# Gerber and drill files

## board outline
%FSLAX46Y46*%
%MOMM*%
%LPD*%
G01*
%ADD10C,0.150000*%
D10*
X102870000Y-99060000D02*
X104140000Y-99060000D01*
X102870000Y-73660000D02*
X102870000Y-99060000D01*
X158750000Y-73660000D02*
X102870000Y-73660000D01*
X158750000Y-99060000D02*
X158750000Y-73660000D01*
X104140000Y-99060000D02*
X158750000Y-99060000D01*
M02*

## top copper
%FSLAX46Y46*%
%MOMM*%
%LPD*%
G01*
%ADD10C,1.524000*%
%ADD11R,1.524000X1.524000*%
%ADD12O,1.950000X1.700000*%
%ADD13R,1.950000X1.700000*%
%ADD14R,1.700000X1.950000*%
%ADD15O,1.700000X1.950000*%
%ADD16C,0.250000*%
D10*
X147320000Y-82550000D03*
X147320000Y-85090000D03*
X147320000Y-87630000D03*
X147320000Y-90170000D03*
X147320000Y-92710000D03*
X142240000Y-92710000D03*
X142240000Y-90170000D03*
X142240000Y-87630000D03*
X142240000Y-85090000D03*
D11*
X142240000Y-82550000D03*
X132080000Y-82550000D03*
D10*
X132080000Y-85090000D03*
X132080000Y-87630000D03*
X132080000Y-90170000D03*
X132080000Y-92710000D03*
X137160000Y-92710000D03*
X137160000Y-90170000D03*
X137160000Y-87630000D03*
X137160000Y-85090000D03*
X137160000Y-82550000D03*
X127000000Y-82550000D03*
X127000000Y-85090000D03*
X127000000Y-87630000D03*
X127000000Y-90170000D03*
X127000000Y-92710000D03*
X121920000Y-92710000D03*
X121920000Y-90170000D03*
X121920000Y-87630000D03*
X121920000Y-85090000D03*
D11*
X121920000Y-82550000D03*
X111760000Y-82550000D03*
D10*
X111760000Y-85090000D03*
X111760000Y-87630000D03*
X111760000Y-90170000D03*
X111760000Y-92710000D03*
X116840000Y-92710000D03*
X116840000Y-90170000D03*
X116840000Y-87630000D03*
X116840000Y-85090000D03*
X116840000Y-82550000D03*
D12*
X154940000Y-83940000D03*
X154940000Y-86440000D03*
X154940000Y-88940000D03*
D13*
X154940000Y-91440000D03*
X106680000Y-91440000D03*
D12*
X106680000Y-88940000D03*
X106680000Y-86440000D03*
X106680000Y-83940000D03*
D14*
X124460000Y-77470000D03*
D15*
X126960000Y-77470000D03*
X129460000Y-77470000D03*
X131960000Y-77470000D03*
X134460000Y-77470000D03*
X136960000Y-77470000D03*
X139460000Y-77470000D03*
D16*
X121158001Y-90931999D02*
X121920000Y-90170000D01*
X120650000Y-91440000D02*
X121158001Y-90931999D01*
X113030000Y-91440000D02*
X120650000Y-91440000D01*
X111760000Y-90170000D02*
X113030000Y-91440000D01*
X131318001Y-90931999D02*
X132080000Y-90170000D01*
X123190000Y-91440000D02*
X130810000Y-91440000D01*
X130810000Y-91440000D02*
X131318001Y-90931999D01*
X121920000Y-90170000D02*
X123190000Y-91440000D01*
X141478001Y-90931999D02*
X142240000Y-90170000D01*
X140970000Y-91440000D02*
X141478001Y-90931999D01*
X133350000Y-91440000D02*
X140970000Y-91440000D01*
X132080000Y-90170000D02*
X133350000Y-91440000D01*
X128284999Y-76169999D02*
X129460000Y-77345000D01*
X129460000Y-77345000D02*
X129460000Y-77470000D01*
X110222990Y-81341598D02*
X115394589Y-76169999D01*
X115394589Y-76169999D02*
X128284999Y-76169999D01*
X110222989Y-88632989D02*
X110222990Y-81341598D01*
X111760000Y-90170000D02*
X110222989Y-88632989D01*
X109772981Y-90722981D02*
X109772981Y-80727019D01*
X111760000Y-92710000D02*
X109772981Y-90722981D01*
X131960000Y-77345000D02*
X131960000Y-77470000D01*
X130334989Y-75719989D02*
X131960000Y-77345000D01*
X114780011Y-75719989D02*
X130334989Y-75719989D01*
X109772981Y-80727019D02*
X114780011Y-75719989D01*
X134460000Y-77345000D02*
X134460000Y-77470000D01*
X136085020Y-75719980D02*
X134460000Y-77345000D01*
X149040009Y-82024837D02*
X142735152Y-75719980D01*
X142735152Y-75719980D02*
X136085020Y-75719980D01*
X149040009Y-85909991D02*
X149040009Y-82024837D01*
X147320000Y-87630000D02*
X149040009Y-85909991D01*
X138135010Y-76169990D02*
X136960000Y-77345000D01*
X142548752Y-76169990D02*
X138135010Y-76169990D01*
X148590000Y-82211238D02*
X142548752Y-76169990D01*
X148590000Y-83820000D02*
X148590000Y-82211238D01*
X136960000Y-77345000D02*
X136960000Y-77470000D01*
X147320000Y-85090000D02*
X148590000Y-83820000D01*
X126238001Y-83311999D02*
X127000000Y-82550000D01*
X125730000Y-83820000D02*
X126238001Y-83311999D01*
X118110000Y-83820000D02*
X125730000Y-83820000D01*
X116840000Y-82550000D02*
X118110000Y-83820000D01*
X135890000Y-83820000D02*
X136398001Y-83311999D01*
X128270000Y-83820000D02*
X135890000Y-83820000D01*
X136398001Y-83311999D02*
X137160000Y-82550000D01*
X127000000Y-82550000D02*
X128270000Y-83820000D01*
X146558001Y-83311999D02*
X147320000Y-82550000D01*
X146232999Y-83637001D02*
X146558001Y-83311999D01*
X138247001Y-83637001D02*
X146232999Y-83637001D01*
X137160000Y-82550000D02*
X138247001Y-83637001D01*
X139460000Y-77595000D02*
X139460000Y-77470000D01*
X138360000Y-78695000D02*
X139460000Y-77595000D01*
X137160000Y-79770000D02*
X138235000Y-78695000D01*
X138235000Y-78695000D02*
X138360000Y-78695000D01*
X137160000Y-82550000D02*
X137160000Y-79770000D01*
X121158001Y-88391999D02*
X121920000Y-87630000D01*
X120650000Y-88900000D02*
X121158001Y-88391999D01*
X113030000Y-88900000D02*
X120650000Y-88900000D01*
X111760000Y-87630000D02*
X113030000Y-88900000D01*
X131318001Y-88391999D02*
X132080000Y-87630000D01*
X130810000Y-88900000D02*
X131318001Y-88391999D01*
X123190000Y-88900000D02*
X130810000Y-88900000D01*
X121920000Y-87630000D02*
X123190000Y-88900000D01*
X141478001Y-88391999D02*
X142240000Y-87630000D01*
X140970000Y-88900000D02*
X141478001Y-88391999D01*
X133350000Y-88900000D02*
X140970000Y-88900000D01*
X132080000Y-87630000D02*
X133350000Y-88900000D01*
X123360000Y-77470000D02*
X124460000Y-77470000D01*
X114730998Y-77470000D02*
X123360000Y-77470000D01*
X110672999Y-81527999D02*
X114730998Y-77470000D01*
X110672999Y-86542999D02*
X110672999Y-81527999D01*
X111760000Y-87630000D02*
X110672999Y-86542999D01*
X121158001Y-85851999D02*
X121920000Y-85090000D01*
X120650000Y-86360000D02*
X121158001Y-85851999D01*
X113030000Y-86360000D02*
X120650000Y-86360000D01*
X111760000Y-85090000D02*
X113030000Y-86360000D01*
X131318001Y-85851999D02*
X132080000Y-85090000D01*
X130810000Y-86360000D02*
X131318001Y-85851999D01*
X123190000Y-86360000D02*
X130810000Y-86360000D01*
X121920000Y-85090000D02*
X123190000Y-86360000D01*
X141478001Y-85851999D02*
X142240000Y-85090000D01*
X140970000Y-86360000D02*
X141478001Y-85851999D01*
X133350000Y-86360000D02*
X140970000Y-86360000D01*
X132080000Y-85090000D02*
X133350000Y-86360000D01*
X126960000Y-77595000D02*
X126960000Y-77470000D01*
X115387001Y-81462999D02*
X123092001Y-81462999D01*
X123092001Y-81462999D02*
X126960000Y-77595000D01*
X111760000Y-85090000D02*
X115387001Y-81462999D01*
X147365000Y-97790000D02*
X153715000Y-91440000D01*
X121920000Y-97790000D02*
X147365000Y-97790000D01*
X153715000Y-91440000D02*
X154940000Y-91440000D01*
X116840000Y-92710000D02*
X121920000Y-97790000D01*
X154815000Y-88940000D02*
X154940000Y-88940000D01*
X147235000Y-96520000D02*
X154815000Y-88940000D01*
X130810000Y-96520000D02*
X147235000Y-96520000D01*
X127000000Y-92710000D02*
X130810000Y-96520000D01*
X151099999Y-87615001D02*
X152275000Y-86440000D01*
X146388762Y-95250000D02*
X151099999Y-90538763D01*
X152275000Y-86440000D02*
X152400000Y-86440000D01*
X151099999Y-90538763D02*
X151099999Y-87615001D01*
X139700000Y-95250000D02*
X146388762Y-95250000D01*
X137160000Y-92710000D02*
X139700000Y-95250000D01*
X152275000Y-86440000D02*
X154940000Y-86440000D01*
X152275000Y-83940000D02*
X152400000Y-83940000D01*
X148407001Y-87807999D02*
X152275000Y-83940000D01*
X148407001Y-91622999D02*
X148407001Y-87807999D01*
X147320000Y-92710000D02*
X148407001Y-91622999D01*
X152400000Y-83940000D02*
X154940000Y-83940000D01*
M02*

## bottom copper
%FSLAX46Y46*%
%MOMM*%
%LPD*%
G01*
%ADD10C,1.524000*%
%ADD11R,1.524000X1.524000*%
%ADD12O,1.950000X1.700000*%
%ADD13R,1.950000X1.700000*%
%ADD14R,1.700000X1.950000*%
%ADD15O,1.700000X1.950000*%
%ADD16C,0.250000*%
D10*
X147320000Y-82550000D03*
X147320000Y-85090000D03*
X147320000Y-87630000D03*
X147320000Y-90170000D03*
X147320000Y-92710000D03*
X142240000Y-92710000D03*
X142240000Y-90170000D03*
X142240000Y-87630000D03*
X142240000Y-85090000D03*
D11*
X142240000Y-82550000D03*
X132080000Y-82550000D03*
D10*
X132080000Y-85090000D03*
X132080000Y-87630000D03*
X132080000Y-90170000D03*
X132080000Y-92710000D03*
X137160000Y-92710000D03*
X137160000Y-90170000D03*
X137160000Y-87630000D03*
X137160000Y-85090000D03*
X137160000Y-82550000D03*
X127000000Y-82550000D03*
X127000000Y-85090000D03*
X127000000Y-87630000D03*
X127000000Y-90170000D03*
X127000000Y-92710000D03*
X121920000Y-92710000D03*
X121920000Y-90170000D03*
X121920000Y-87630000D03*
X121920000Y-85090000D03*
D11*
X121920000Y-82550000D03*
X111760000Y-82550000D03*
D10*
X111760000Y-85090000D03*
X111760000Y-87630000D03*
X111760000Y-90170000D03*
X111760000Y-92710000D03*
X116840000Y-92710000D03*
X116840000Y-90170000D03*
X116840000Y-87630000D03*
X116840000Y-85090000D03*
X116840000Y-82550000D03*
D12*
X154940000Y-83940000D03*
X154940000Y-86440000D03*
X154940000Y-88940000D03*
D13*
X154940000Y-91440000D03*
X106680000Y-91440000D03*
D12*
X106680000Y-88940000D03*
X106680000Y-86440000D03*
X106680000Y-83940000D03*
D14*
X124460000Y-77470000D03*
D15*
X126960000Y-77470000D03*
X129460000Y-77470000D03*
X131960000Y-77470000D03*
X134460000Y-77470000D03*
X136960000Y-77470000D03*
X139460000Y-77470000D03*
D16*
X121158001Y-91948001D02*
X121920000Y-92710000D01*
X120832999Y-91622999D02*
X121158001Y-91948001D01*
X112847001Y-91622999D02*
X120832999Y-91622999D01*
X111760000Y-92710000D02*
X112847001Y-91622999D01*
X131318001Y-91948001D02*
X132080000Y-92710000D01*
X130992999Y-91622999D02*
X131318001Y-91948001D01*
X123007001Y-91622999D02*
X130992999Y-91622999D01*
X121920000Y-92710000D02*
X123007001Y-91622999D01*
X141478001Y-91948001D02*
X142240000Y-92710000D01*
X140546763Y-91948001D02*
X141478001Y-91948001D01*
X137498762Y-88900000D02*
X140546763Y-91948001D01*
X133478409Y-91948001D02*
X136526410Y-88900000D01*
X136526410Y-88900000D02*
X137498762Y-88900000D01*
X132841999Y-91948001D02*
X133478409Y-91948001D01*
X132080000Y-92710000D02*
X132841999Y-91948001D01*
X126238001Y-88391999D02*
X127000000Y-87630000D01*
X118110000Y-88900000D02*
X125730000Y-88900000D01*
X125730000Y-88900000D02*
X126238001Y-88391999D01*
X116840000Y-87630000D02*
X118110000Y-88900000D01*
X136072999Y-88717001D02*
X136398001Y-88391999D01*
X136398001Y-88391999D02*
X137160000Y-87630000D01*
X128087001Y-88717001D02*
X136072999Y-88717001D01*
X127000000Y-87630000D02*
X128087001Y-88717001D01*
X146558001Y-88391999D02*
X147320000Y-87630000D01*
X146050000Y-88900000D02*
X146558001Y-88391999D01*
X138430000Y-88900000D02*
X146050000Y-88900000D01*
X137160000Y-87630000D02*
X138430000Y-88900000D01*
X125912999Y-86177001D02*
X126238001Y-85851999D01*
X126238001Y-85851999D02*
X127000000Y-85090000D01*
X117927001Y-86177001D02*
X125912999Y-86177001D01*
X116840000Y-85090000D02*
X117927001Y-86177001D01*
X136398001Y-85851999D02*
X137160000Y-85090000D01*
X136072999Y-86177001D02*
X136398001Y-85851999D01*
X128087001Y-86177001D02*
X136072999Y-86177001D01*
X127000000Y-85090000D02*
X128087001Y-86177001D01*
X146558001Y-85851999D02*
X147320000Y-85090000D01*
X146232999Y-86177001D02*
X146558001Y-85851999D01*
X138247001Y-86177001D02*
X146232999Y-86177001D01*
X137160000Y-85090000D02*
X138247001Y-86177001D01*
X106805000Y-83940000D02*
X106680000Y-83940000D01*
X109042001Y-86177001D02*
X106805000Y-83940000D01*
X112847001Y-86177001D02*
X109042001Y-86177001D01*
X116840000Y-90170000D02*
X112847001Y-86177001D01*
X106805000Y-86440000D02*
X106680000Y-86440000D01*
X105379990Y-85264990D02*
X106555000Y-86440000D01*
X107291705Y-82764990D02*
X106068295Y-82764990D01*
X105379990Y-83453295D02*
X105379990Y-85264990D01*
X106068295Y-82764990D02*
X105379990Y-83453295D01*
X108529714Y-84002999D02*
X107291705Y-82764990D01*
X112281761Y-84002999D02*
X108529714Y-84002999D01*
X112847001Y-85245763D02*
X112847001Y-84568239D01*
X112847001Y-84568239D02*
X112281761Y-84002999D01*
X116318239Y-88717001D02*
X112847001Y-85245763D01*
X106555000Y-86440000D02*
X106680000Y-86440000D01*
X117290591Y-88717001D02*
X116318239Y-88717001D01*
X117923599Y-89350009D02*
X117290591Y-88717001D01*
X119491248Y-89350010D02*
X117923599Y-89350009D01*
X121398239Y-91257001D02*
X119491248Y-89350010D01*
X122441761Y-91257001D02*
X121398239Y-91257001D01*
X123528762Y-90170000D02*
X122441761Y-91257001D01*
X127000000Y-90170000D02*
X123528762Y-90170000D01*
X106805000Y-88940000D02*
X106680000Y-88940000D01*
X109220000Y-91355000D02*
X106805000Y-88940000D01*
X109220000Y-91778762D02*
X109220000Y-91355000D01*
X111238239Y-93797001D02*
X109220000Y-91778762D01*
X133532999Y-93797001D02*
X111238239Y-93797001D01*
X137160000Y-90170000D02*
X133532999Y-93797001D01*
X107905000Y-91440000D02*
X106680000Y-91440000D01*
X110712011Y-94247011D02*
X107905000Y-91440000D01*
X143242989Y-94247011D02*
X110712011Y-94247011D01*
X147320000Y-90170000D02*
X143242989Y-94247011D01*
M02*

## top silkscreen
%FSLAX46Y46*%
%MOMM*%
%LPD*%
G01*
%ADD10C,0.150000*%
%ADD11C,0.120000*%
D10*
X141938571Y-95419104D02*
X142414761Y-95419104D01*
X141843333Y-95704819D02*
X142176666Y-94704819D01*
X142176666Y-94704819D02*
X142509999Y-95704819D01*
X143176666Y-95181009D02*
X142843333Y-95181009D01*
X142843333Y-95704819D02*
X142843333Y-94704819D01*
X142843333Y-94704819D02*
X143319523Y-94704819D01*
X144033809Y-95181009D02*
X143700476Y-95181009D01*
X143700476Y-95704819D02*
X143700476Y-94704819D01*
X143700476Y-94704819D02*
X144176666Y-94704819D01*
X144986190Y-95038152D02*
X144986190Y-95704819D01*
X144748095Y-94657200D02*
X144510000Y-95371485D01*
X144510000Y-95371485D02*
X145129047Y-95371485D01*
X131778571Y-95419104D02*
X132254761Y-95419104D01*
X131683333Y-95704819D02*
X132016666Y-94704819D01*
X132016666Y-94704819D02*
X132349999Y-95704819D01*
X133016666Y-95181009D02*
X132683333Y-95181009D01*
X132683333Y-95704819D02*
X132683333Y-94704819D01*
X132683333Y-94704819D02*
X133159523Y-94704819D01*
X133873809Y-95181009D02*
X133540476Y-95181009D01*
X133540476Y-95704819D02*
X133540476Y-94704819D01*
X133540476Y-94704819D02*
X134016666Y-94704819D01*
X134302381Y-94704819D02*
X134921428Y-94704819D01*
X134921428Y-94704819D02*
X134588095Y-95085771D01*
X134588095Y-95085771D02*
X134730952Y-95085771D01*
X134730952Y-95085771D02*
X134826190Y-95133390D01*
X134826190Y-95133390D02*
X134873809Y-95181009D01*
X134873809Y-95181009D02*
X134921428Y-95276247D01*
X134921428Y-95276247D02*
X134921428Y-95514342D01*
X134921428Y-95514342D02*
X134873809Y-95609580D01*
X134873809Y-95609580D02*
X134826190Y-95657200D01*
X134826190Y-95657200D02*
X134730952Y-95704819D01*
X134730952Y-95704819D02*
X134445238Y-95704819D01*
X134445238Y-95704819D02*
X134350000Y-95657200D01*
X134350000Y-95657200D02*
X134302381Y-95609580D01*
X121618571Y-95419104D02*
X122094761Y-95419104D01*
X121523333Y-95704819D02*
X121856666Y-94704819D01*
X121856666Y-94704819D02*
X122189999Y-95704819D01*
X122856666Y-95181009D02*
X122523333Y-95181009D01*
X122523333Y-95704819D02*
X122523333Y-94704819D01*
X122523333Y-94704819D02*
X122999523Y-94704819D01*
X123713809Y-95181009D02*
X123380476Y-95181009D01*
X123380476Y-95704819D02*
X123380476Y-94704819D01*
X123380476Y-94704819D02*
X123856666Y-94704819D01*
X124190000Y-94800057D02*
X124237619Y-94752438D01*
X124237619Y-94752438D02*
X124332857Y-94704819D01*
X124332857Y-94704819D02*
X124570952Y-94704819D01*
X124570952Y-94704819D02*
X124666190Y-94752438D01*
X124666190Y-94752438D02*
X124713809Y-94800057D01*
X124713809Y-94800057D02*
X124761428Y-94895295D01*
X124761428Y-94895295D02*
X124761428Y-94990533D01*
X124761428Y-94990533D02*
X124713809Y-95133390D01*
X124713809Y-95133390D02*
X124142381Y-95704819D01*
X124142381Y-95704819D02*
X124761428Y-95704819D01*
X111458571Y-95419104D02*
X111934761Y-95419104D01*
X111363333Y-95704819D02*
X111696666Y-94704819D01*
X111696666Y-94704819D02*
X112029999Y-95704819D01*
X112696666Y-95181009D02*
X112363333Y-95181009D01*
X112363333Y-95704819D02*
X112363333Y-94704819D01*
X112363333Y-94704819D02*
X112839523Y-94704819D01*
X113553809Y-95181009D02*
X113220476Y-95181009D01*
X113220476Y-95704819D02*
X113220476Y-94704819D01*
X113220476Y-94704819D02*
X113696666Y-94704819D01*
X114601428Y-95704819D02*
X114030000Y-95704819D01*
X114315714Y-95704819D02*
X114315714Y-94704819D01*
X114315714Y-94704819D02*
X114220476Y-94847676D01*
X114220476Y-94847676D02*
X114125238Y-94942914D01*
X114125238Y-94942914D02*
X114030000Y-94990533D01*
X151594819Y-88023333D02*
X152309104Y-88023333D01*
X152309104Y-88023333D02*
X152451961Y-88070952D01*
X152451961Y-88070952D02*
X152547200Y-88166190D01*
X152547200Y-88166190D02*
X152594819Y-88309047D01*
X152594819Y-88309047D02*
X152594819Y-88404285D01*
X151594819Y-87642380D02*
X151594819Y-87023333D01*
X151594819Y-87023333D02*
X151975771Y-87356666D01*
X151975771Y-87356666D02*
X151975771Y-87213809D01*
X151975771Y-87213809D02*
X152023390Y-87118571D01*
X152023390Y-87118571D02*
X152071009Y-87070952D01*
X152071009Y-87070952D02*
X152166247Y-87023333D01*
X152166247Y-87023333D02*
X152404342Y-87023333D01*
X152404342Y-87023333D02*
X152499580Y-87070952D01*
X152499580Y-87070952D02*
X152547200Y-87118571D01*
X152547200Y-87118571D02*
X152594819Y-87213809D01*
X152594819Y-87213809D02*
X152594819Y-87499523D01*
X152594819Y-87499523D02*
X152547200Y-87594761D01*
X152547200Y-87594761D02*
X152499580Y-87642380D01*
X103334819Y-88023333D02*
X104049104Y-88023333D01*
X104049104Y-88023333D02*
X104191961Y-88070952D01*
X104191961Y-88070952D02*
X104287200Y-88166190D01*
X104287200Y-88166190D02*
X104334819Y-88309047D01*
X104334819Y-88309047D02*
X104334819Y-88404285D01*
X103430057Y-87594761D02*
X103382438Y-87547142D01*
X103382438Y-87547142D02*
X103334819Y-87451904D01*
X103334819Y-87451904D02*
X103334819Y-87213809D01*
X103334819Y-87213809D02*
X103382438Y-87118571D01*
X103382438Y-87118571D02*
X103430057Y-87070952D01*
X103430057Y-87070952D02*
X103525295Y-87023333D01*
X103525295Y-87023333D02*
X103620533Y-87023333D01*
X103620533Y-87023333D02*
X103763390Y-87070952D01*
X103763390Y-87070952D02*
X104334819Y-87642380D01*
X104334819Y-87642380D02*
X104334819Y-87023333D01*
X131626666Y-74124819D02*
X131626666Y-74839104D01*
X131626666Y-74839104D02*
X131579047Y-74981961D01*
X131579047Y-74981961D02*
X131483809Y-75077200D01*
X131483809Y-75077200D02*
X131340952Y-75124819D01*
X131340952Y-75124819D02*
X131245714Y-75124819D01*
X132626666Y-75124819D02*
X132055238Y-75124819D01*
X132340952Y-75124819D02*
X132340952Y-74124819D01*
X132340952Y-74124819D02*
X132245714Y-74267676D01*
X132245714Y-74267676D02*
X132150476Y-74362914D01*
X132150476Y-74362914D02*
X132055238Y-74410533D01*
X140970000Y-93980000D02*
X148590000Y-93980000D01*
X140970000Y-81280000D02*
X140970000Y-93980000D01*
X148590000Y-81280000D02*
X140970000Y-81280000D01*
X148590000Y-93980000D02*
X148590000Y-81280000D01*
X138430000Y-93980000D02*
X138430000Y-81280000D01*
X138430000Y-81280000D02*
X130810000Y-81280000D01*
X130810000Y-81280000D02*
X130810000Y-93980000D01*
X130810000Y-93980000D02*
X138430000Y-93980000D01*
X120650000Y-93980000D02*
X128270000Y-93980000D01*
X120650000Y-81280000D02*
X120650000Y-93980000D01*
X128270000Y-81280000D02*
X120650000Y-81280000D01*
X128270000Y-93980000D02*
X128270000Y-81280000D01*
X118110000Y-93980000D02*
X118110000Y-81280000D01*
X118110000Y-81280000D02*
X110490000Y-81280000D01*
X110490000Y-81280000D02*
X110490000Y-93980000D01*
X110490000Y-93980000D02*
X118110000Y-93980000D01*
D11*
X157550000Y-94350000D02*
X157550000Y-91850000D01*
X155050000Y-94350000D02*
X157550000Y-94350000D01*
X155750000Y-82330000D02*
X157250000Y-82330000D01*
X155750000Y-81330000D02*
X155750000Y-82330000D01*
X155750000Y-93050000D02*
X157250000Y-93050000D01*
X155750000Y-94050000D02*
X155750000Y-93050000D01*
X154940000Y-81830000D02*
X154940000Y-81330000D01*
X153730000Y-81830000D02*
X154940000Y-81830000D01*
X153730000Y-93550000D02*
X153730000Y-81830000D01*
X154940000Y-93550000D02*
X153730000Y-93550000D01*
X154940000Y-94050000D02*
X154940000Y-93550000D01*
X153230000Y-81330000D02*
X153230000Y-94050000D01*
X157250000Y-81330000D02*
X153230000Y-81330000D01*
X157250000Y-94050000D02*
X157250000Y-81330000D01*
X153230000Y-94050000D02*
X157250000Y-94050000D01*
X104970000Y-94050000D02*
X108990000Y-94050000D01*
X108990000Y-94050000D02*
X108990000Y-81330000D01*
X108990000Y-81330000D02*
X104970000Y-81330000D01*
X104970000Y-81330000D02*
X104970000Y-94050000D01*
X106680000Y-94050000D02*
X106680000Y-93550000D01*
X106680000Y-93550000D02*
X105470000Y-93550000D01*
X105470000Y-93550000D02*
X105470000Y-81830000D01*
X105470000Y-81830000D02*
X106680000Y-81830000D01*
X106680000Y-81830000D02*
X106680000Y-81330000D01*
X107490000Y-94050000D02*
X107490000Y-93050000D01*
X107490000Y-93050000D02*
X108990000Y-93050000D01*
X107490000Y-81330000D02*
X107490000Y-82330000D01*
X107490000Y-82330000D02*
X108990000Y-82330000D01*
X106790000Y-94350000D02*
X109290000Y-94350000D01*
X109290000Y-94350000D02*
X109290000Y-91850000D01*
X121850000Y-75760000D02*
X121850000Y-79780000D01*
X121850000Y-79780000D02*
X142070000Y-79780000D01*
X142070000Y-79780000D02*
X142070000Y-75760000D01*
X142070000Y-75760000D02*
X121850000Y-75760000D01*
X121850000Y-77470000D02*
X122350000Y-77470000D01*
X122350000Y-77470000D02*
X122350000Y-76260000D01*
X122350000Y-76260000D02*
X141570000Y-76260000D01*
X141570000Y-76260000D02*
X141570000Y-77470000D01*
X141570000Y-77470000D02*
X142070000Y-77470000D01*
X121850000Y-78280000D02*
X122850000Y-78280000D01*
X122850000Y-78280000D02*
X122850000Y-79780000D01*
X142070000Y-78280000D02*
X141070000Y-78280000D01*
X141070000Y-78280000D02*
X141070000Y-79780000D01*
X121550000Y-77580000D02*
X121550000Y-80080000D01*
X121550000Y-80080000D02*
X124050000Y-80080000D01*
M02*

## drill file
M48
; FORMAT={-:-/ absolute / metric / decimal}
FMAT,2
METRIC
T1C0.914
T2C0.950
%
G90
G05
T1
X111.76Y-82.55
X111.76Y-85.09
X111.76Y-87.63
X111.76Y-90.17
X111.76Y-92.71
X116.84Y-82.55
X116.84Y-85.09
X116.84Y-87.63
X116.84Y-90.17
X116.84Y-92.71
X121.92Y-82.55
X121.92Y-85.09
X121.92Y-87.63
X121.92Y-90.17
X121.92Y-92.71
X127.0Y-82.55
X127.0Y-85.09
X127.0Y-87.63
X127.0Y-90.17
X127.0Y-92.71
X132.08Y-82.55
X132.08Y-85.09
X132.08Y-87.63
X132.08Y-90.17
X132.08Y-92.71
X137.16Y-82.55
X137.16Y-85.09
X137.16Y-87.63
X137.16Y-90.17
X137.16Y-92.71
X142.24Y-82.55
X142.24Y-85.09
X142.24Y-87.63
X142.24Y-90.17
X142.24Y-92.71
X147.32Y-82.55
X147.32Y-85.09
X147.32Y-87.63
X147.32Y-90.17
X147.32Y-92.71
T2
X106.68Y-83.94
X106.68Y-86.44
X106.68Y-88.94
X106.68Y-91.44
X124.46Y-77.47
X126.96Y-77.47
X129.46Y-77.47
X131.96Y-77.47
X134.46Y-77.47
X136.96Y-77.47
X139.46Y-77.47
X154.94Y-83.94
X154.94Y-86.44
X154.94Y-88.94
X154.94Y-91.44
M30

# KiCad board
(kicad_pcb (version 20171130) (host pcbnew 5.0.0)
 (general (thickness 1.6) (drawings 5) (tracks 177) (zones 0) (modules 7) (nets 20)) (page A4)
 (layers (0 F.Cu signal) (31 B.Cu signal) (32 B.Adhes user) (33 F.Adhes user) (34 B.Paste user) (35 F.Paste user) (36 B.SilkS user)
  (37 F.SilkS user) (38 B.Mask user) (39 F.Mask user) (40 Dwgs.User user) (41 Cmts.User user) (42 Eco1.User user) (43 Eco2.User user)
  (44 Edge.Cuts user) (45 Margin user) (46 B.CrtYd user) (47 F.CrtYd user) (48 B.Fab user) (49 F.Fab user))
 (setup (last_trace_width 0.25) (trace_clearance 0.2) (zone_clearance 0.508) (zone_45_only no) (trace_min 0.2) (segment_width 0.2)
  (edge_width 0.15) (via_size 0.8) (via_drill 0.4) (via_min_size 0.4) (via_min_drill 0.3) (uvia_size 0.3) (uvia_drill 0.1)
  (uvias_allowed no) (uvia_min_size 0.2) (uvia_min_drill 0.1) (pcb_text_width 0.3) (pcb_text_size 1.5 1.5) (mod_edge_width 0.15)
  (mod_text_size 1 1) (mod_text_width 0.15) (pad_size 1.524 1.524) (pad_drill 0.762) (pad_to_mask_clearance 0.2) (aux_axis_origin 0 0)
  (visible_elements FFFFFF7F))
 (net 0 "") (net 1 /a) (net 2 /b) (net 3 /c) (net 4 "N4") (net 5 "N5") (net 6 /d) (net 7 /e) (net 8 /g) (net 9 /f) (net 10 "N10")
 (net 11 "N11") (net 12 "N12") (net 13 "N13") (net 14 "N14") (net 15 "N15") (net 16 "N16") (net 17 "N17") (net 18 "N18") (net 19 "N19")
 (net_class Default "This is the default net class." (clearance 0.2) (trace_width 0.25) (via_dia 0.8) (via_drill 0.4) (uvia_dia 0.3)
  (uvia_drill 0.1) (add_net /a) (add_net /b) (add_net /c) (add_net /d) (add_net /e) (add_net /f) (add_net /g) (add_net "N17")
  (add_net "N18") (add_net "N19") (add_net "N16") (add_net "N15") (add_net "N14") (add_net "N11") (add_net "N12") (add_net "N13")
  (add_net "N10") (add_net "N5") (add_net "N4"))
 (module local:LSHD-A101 (layer F.Cu) (at 144.78 87.63 90)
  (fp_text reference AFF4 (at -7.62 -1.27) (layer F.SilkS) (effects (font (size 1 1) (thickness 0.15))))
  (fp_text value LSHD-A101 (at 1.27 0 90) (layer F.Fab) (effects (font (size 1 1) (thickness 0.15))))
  (fp_line (start -6.35 -3.81) (end -6.35 3.81) (layer F.SilkS) (width 0.15))
  (fp_line (start 6.35 -3.81) (end -6.35 -3.81) (layer F.SilkS) (width 0.15))
  (fp_line (start 6.35 3.81) (end 6.35 -3.81) (layer F.SilkS) (width 0.15))
  (fp_line (start -6.35 3.81) (end 6.35 3.81) (layer F.SilkS) (width 0.15))
  (pad 10 thru_hole circle (at 5.08 2.54) (size 1.524 1.524) (drill 0.9144) (layers *.Cu *.Mask) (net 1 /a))
  (pad 9 thru_hole circle (at 2.54 2.54) (size 1.524 1.524) (drill 0.9144) (layers *.Cu *.Mask) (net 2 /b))
  (pad 8 thru_hole circle (at 0 2.54) (size 1.524 1.524) (drill 0.9144) (layers *.Cu *.Mask) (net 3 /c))
  (pad 7 thru_hole circle (at -2.54 2.54) (size 1.524 1.524) (drill 0.9144) (layers *.Cu *.Mask) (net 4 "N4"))
  (pad 6 thru_hole circle (at -5.08 2.54) (size 1.524 1.524) (drill 0.9144) (layers *.Cu *.Mask) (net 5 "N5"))
  (pad 5 thru_hole circle (at -5.08 -2.54) (size 1.524 1.524) (drill 0.9144) (layers *.Cu *.Mask) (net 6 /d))
  (pad 4 thru_hole circle (at -2.54 -2.54) (size 1.524 1.524) (drill 0.9144) (layers *.Cu *.Mask) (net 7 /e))
  (pad 3 thru_hole circle (at 0 -2.54) (size 1.524 1.524) (drill 0.9144) (layers *.Cu *.Mask) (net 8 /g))
  (pad 2 thru_hole circle (at 2.54 -2.54) (size 1.524 1.524) (drill 0.9144) (layers *.Cu *.Mask) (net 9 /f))
  (pad 1 thru_hole rect (at 5.08 -2.54) (size 1.524 1.524) (drill 0.9144) (layers *.Cu *.Mask) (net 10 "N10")))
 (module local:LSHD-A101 (layer F.Cu) (at 134.62 87.63 90)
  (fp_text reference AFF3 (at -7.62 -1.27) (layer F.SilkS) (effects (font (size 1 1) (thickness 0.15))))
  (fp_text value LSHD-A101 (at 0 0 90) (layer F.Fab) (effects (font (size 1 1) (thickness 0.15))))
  (fp_line (start -6.35 3.81) (end 6.35 3.81) (layer F.SilkS) (width 0.15))
  (fp_line (start 6.35 3.81) (end 6.35 -3.81) (layer F.SilkS) (width 0.15))
  (fp_line (start 6.35 -3.81) (end -6.35 -3.81) (layer F.SilkS) (width 0.15))
  (fp_line (start -6.35 -3.81) (end -6.35 3.81) (layer F.SilkS) (width 0.15))
  (pad 1 thru_hole rect (at 5.08 -2.54) (size 1.524 1.524) (drill 0.9144) (layers *.Cu *.Mask) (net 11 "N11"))
  (pad 2 thru_hole circle (at 2.54 -2.54) (size 1.524 1.524) (drill 0.9144) (layers *.Cu *.Mask) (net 9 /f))
  (pad 3 thru_hole circle (at 0 -2.54) (size 1.524 1.524) (drill 0.9144) (layers *.Cu *.Mask) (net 8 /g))
  (pad 4 thru_hole circle (at -2.54 -2.54) (size 1.524 1.524) (drill 0.9144) (layers *.Cu *.Mask) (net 7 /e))
  (pad 5 thru_hole circle (at -5.08 -2.54) (size 1.524 1.524) (drill 0.9144) (layers *.Cu *.Mask) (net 6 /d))
  (pad 6 thru_hole circle (at -5.08 2.54) (size 1.524 1.524) (drill 0.9144) (layers *.Cu *.Mask) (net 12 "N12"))
  (pad 7 thru_hole circle (at -2.54 2.54) (size 1.524 1.524) (drill 0.9144) (layers *.Cu *.Mask) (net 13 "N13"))
  (pad 8 thru_hole circle (at 0 2.54) (size 1.524 1.524) (drill 0.9144) (layers *.Cu *.Mask) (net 3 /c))
  (pad 9 thru_hole circle (at 2.54 2.54) (size 1.524 1.524) (drill 0.9144) (layers *.Cu *.Mask) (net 2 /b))
  (pad 10 thru_hole circle (at 5.08 2.54) (size 1.524 1.524) (drill 0.9144) (layers *.Cu *.Mask) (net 1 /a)))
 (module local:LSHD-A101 (layer F.Cu) (at 124.46 87.63 90)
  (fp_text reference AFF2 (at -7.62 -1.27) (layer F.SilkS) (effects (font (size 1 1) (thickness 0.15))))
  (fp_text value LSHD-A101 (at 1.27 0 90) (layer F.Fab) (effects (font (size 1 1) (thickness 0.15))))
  (fp_line (start -6.35 -3.81) (end -6.35 3.81) (layer F.SilkS) (width 0.15))
  (fp_line (start 6.35 -3.81) (end -6.35 -3.81) (layer F.SilkS) (width 0.15))
  (fp_line (start 6.35 3.81) (end 6.35 -3.81) (layer F.SilkS) (width 0.15))
  (fp_line (start -6.35 3.81) (end 6.35 3.81) (layer F.SilkS) (width 0.15))
  (pad 10 thru_hole circle (at 5.08 2.54) (size 1.524 1.524) (drill 0.9144) (layers *.Cu *.Mask) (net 1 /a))
  (pad 9 thru_hole circle (at 2.54 2.54) (size 1.524 1.524) (drill 0.9144) (layers *.Cu *.Mask) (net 2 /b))
  (pad 8 thru_hole circle (at 0 2.54) (size 1.524 1.524) (drill 0.9144) (layers *.Cu *.Mask) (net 3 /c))
  (pad 7 thru_hole circle (at -2.54 2.54) (size 1.524 1.524) (drill 0.9144) (layers *.Cu *.Mask) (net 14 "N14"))
  (pad 6 thru_hole circle (at -5.08 2.54) (size 1.524 1.524) (drill 0.9144) (layers *.Cu *.Mask) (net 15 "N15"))
  (pad 5 thru_hole circle (at -5.08 -2.54) (size 1.524 1.524) (drill 0.9144) (layers *.Cu *.Mask) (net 6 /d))
  (pad 4 thru_hole circle (at -2.54 -2.54) (size 1.524 1.524) (drill 0.9144) (layers *.Cu *.Mask) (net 7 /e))
  (pad 3 thru_hole circle (at 0 -2.54) (size 1.524 1.524) (drill 0.9144) (layers *.Cu *.Mask) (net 8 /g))
  (pad 2 thru_hole circle (at 2.54 -2.54) (size 1.524 1.524) (drill 0.9144) (layers *.Cu *.Mask) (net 9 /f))
  (pad 1 thru_hole rect (at 5.08 -2.54) (size 1.524 1.524) (drill 0.9144) (layers *.Cu *.Mask) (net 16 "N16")))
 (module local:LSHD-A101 (layer F.Cu) (at 114.3 87.63 90)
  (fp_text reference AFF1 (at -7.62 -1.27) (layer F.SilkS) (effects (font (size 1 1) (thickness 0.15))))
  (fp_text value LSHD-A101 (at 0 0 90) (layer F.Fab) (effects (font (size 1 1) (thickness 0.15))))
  (fp_line (start -6.35 3.81) (end 6.35 3.81) (layer F.SilkS) (width 0.15))
  (fp_line (start 6.35 3.81) (end 6.35 -3.81) (layer F.SilkS) (width 0.15))
  (fp_line (start 6.35 -3.81) (end -6.35 -3.81) (layer F.SilkS) (width 0.15))
  (fp_line (start -6.35 -3.81) (end -6.35 3.81) (layer F.SilkS) (width 0.15))
  (pad 1 thru_hole rect (at 5.08 -2.54) (size 1.524 1.524) (drill 0.9144) (layers *.Cu *.Mask) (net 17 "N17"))
  (pad 2 thru_hole circle (at 2.54 -2.54) (size 1.524 1.524) (drill 0.9144) (layers *.Cu *.Mask) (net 9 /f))
  (pad 3 thru_hole circle (at 0 -2.54) (size 1.524 1.524) (drill 0.9144) (layers *.Cu *.Mask) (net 8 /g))
  (pad 4 thru_hole circle (at -2.54 -2.54) (size 1.524 1.524) (drill 0.9144) (layers *.Cu *.Mask) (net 7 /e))
  (pad 5 thru_hole circle (at -5.08 -2.54) (size 1.524 1.524) (drill 0.9144) (layers *.Cu *.Mask) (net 6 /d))
  (pad 6 thru_hole circle (at -5.08 2.54) (size 1.524 1.524) (drill 0.9144) (layers *.Cu *.Mask) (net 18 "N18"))
  (pad 7 thru_hole circle (at -2.54 2.54) (size 1.524 1.524) (drill 0.9144) (layers *.Cu *.Mask) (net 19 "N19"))
  (pad 8 thru_hole circle (at 0 2.54) (size 1.524 1.524) (drill 0.9144) (layers *.Cu *.Mask) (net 3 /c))
  (pad 9 thru_hole circle (at 2.54 2.54) (size 1.524 1.524) (drill 0.9144) (layers *.Cu *.Mask) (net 2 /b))
  (pad 10 thru_hole circle (at 5.08 2.54) (size 1.524 1.524) (drill 0.9144) (layers *.Cu *.Mask) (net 1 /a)))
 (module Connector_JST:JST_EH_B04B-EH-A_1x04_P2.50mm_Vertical (layer F.Cu) (at 154.94 91.44 90)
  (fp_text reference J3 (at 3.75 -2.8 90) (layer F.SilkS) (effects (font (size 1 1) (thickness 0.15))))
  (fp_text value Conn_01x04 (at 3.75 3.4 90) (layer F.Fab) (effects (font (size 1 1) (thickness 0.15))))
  (fp_line (start -2.91 2.61) (end -0.41 2.61) (layer F.SilkS) (width 0.12))
  (fp_line (start -2.91 0.11) (end -2.91 2.61) (layer F.SilkS) (width 0.12))
  (fp_line (start 9.11 0.81) (end 9.11 2.31) (layer F.SilkS) (width 0.12))
  (fp_line (start 10.11 0.81) (end 9.11 0.81) (layer F.SilkS) (width 0.12))
  (fp_line (start -1.61 0.81) (end -1.61 2.31) (layer F.SilkS) (width 0.12))
  (fp_line (start -2.61 0.81) (end -1.61 0.81) (layer F.SilkS) (width 0.12))
  (fp_line (start 9.61 0) (end 10.11 0) (layer F.SilkS) (width 0.12))
  (fp_line (start 9.61 -1.21) (end 9.61 0) (layer F.SilkS) (width 0.12))
  (fp_line (start -2.11 -1.21) (end 9.61 -1.21) (layer F.SilkS) (width 0.12))
  (fp_line (start -2.11 0) (end -2.11 -1.21) (layer F.SilkS) (width 0.12))
  (fp_line (start -2.61 0) (end -2.11 0) (layer F.SilkS) (width 0.12))
  (fp_line (start 10.11 -1.71) (end -2.61 -1.71) (layer F.SilkS) (width 0.12))
  (fp_line (start 10.11 2.31) (end 10.11 -1.71) (layer F.SilkS) (width 0.12))
  (fp_line (start -2.61 2.31) (end 10.11 2.31) (layer F.SilkS) (width 0.12))
  (fp_line (start -2.61 -1.71) (end -2.61 2.31) (layer F.SilkS) (width 0.12))
  (pad 4 thru_hole oval (at 7.5 0 90) (size 1.7 1.95) (drill 0.95) (layers *.Cu *.Mask) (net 5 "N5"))
  (pad 3 thru_hole oval (at 5 0 90) (size 1.7 1.95) (drill 0.95) (layers *.Cu *.Mask) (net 12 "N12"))
  (pad 2 thru_hole oval (at 2.5 0 90) (size 1.7 1.95) (drill 0.95) (layers *.Cu *.Mask) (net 15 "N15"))
  (pad 1 thru_hole rect (at 0 0 90) (size 1.7 1.95) (drill 0.95) (layers *.Cu *.Mask) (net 18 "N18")))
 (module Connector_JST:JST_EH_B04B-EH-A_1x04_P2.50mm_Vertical (layer F.Cu) (at 106.68 91.44 90)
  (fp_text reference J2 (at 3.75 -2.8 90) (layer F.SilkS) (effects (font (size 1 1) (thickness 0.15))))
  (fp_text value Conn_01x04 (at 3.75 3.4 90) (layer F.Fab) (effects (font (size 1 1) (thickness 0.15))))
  (fp_line (start -2.61 -1.71) (end -2.61 2.31) (layer F.SilkS) (width 0.12))
  (fp_line (start -2.61 2.31) (end 10.11 2.31) (layer F.SilkS) (width 0.12))
  (fp_line (start 10.11 2.31) (end 10.11 -1.71) (layer F.SilkS) (width 0.12))
  (fp_line (start 10.11 -1.71) (end -2.61 -1.71) (layer F.SilkS) (width 0.12))
  (fp_line (start -2.61 0) (end -2.11 0) (layer F.SilkS) (width 0.12))
  (fp_line (start -2.11 0) (end -2.11 -1.21) (layer F.SilkS) (width 0.12))
  (fp_line (start -2.11 -1.21) (end 9.61 -1.21) (layer F.SilkS) (width 0.12))
  (fp_line (start 9.61 -1.21) (end 9.61 0) (layer F.SilkS) (width 0.12))
  (fp_line (start 9.61 0) (end 10.11 0) (layer F.SilkS) (width 0.12))
  (fp_line (start -2.61 0.81) (end -1.61 0.81) (layer F.SilkS) (width 0.12))
  (fp_line (start -1.61 0.81) (end -1.61 2.31) (layer F.SilkS) (width 0.12))
  (fp_line (start 10.11 0.81) (end 9.11 0.81) (layer F.SilkS) (width 0.12))
  (fp_line (start 9.11 0.81) (end 9.11 2.31) (layer F.SilkS) (width 0.12))
  (fp_line (start -2.91 0.11) (end -2.91 2.61) (layer F.SilkS) (width 0.12))
  (fp_line (start -2.91 2.61) (end -0.41 2.61) (layer F.SilkS) (width 0.12))
  (pad 1 thru_hole rect (at 0 0 90) (size 1.7 1.95) (drill 0.95) (layers *.Cu *.Mask) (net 4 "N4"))
  (pad 2 thru_hole oval (at 2.5 0 90) (size 1.7 1.95) (drill 0.95) (layers *.Cu *.Mask) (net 13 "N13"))
  (pad 3 thru_hole oval (at 5 0 90) (size 1.7 1.95) (drill 0.95) (layers *.Cu *.Mask) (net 14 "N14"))
  (pad 4 thru_hole oval (at 7.5 0 90) (size 1.7 1.95) (drill 0.95) (layers *.Cu *.Mask) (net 19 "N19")))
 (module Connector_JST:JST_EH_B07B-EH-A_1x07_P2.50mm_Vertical (layer F.Cu) (at 124.46 77.47)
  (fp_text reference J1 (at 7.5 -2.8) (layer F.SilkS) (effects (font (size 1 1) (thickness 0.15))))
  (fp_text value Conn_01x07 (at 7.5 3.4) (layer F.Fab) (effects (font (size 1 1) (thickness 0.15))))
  (fp_line (start -2.61 -1.71) (end -2.61 2.31) (layer F.SilkS) (width 0.12))
  (fp_line (start -2.61 2.31) (end 17.61 2.31) (layer F.SilkS) (width 0.12))
  (fp_line (start 17.61 2.31) (end 17.61 -1.71) (layer F.SilkS) (width 0.12))
  (fp_line (start 17.61 -1.71) (end -2.61 -1.71) (layer F.SilkS) (width 0.12))
  (fp_line (start -2.61 0) (end -2.11 0) (layer F.SilkS) (width 0.12))
  (fp_line (start -2.11 0) (end -2.11 -1.21) (layer F.SilkS) (width 0.12))
  (fp_line (start -2.11 -1.21) (end 17.11 -1.21) (layer F.SilkS) (width 0.12))
  (fp_line (start 17.11 -1.21) (end 17.11 0) (layer F.SilkS) (width 0.12))
  (fp_line (start 17.11 0) (end 17.61 0) (layer F.SilkS) (width 0.12))
  (fp_line (start -2.61 0.81) (end -1.61 0.81) (layer F.SilkS) (width 0.12))
  (fp_line (start -1.61 0.81) (end -1.61 2.31) (layer F.SilkS) (width 0.12))
  (fp_line (start 17.61 0.81) (end 16.61 0.81) (layer F.SilkS) (width 0.12))
  (fp_line (start 16.61 0.81) (end 16.61 2.31) (layer F.SilkS) (width 0.12))
  (fp_line (start -2.91 0.11) (end -2.91 2.61) (layer F.SilkS) (width 0.12))
  (fp_line (start -2.91 2.61) (end -0.41 2.61) (layer F.SilkS) (width 0.12))
  (pad 1 thru_hole rect (at 0 0) (size 1.7 1.95) (drill 0.95) (layers *.Cu *.Mask) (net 8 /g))
  (pad 2 thru_hole oval (at 2.5 0) (size 1.7 1.95) (drill 0.95) (layers *.Cu *.Mask) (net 9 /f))
  (pad 3 thru_hole oval (at 5 0) (size 1.7 1.95) (drill 0.95) (layers *.Cu *.Mask) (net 7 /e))
  (pad 4 thru_hole oval (at 7.5 0) (size 1.7 1.95) (drill 0.95) (layers *.Cu *.Mask) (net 6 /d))
  (pad 5 thru_hole oval (at 10 0) (size 1.7 1.95) (drill 0.95) (layers *.Cu *.Mask) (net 3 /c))
  (pad 6 thru_hole oval (at 12.5 0) (size 1.7 1.95) (drill 0.95) (layers *.Cu *.Mask) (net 2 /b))
  (pad 7 thru_hole oval (at 15 0) (size 1.7 1.95) (drill 0.95) (layers *.Cu *.Mask) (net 1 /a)))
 (gr_line (start 102.87 99.06) (end 104.14 99.06) (layer Edge.Cuts) (width 0.15))
 (gr_line (start 102.87 73.66) (end 102.87 99.06) (layer Edge.Cuts) (width 0.15))
 (gr_line (start 158.75 73.66) (end 102.87 73.66) (layer Edge.Cuts) (width 0.15))
 (gr_line (start 158.75 99.06) (end 158.75 73.66) (layer Edge.Cuts) (width 0.15))
 (gr_line (start 104.14 99.06) (end 158.75 99.06) (layer Edge.Cuts) (width 0.15))
 (segment (start 121.158001 90.931999) (end 121.92 90.17) (width 0.25) (layer F.Cu) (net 7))
 (segment (start 120.65 91.44) (end 121.158001 90.931999) (width 0.25) (layer F.Cu) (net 7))
 (segment (start 113.03 91.44) (end 120.65 91.44) (width 0.25) (layer F.Cu) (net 7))
 (segment (start 111.76 90.17) (end 113.03 91.44) (width 0.25) (layer F.Cu) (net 7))
 (segment (start 131.318001 90.931999) (end 132.08 90.17) (width 0.25) (layer F.Cu) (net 7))
 (segment (start 123.19 91.44) (end 130.81 91.44) (width 0.25) (layer F.Cu) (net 7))
 (segment (start 130.81 91.44) (end 131.318001 90.931999) (width 0.25) (layer F.Cu) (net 7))
 (segment (start 121.92 90.17) (end 123.19 91.44) (width 0.25) (layer F.Cu) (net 7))
 (segment (start 141.478001 90.931999) (end 142.24 90.17) (width 0.25) (layer F.Cu) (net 7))
 (segment (start 140.97 91.44) (end 141.478001 90.931999) (width 0.25) (layer F.Cu) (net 7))
 (segment (start 133.35 91.44) (end 140.97 91.44) (width 0.25) (layer F.Cu) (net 7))
 (segment (start 132.08 90.17) (end 133.35 91.44) (width 0.25) (layer F.Cu) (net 7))
 (segment (start 128.284999 76.169999) (end 129.46 77.345) (width 0.25) (layer F.Cu) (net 7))
 (segment (start 129.46 77.345) (end 129.46 77.47) (width 0.25) (layer F.Cu) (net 7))
 (segment (start 110.22299 81.341598) (end 115.394589 76.169999) (width 0.25) (layer F.Cu) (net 7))
 (segment (start 115.394589 76.169999) (end 128.284999 76.169999) (width 0.25) (layer F.Cu) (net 7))
 (segment (start 110.222989 88.632989) (end 110.22299 81.341598) (width 0.25) (layer F.Cu) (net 7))
 (segment (start 111.76 90.17) (end 110.222989 88.632989) (width 0.25) (layer F.Cu) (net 7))
 (segment (start 121.158001 91.948001) (end 121.92 92.71) (width 0.25) (layer B.Cu) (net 6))
 (segment (start 120.832999 91.622999) (end 121.158001 91.948001) (width 0.25) (layer B.Cu) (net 6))
 (segment (start 112.847001 91.622999) (end 120.832999 91.622999) (width 0.25) (layer B.Cu) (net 6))
 (segment (start 111.76 92.71) (end 112.847001 91.622999) (width 0.25) (layer B.Cu) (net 6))
 (segment (start 131.318001 91.948001) (end 132.08 92.71) (width 0.25) (layer B.Cu) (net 6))
 (segment (start 130.992999 91.622999) (end 131.318001 91.948001) (width 0.25) (layer B.Cu) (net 6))
 (segment (start 123.007001 91.622999) (end 130.992999 91.622999) (width 0.25) (layer B.Cu) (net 6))
 (segment (start 121.92 92.71) (end 123.007001 91.622999) (width 0.25) (layer B.Cu) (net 6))
 (segment (start 141.478001 91.948001) (end 142.24 92.71) (width 0.25) (layer B.Cu) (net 6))
 (segment (start 140.546763 91.948001) (end 141.478001 91.948001) (width 0.25) (layer B.Cu) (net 6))
 (segment (start 137.498762 88.9) (end 140.546763 91.948001) (width 0.25) (layer B.Cu) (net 6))
 (segment (start 133.478409 91.948001) (end 136.52641 88.9) (width 0.25) (layer B.Cu) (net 6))
 (segment (start 136.52641 88.9) (end 137.498762 88.9) (width 0.25) (layer B.Cu) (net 6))
 (segment (start 132.841999 91.948001) (end 133.478409 91.948001) (width 0.25) (layer B.Cu) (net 6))
 (segment (start 132.08 92.71) (end 132.841999 91.948001) (width 0.25) (layer B.Cu) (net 6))
 (segment (start 109.772981 90.722981) (end 109.772981 80.727019) (width 0.25) (layer F.Cu) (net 6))
 (segment (start 111.76 92.71) (end 109.772981 90.722981) (width 0.25) (layer F.Cu) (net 6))
 (segment (start 131.96 77.345) (end 131.96 77.47) (width 0.25) (layer F.Cu) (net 6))
 (segment (start 130.334989 75.719989) (end 131.96 77.345) (width 0.25) (layer F.Cu) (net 6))
 (segment (start 114.780011 75.719989) (end 130.334989 75.719989) (width 0.25) (layer F.Cu) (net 6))
 (segment (start 109.772981 80.727019) (end 114.780011 75.719989) (width 0.25) (layer F.Cu) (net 6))
 (segment (start 126.238001 88.391999) (end 127 87.63) (width 0.25) (layer B.Cu) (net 3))
 (segment (start 118.11 88.9) (end 125.73 88.9) (width 0.25) (layer B.Cu) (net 3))
 (segment (start 125.73 88.9) (end 126.238001 88.391999) (width 0.25) (layer B.Cu) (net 3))
 (segment (start 116.84 87.63) (end 118.11 88.9) (width 0.25) (layer B.Cu) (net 3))
 (segment (start 136.072999 88.717001) (end 136.398001 88.391999) (width 0.25) (layer B.Cu) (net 3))
 (segment (start 136.398001 88.391999) (end 137.16 87.63) (width 0.25) (layer B.Cu) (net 3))
 (segment (start 128.087001 88.717001) (end 136.072999 88.717001) (width 0.25) (layer B.Cu) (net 3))
 (segment (start 127 87.63) (end 128.087001 88.717001) (width 0.25) (layer B.Cu) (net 3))
 (segment (start 146.558001 88.391999) (end 147.32 87.63) (width 0.25) (layer B.Cu) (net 3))
 (segment (start 146.05 88.9) (end 146.558001 88.391999) (width 0.25) (layer B.Cu) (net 3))
 (segment (start 138.43 88.9) (end 146.05 88.9) (width 0.25) (layer B.Cu) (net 3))
 (segment (start 137.16 87.63) (end 138.43 88.9) (width 0.25) (layer B.Cu) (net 3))
 (segment (start 134.46 77.345) (end 134.46 77.47) (width 0.25) (layer F.Cu) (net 3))
 (segment (start 136.08502 75.71998) (end 134.46 77.345) (width 0.25) (layer F.Cu) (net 3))
 (segment (start 149.040009 82.024837) (end 142.735152 75.71998) (width 0.25) (layer F.Cu) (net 3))
 (segment (start 142.735152 75.71998) (end 136.08502 75.71998) (width 0.25) (layer F.Cu) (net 3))
 (segment (start 149.040009 85.909991) (end 149.040009 82.024837) (width 0.25) (layer F.Cu) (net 3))
 (segment (start 147.32 87.63) (end 149.040009 85.909991) (width 0.25) (layer F.Cu) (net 3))
 (segment (start 125.912999 86.177001) (end 126.238001 85.851999) (width 0.25) (layer B.Cu) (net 2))
 (segment (start 126.238001 85.851999) (end 127 85.09) (width 0.25) (layer B.Cu) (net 2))
 (segment (start 117.927001 86.177001) (end 125.912999 86.177001) (width 0.25) (layer B.Cu) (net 2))
 (segment (start 116.84 85.09) (end 117.927001 86.177001) (width 0.25) (layer B.Cu) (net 2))
 (segment (start 136.398001 85.851999) (end 137.16 85.09) (width 0.25) (layer B.Cu) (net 2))
 (segment (start 136.072999 86.177001) (end 136.398001 85.851999) (width 0.25) (layer B.Cu) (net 2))
 (segment (start 128.087001 86.177001) (end 136.072999 86.177001) (width 0.25) (layer B.Cu) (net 2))
 (segment (start 127 85.09) (end 128.087001 86.177001) (width 0.25) (layer B.Cu) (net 2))
 (segment (start 146.558001 85.851999) (end 147.32 85.09) (width 0.25) (layer B.Cu) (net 2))
 (segment (start 146.232999 86.177001) (end 146.558001 85.851999) (width 0.25) (layer B.Cu) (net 2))
 (segment (start 138.247001 86.177001) (end 146.232999 86.177001) (width 0.25) (layer B.Cu) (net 2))
 (segment (start 137.16 85.09) (end 138.247001 86.177001) (width 0.25) (layer B.Cu) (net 2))
 (segment (start 138.13501 76.16999) (end 136.96 77.345) (width 0.25) (layer F.Cu) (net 2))
 (segment (start 142.548752 76.16999) (end 138.13501 76.16999) (width 0.25) (layer F.Cu) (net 2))
 (segment (start 148.59 82.211238) (end 142.548752 76.16999) (width 0.25) (layer F.Cu) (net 2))
 (segment (start 148.59 83.82) (end 148.59 82.211238) (width 0.25) (layer F.Cu) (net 2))
 (segment (start 136.96 77.345) (end 136.96 77.47) (width 0.25) (layer F.Cu) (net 2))
 (segment (start 147.32 85.09) (end 148.59 83.82) (width 0.25) (layer F.Cu) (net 2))
 (segment (start 126.238001 83.311999) (end 127 82.55) (width 0.25) (layer F.Cu) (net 1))
 (segment (start 125.73 83.82) (end 126.238001 83.311999) (width 0.25) (layer F.Cu) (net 1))
 (segment (start 118.11 83.82) (end 125.73 83.82) (width 0.25) (layer F.Cu) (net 1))
 (segment (start 116.84 82.55) (end 118.11 83.82) (width 0.25) (layer F.Cu) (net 1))
 (segment (start 135.89 83.82) (end 136.398001 83.311999) (width 0.25) (layer F.Cu) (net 1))
 (segment (start 128.27 83.82) (end 135.89 83.82) (width 0.25) (layer F.Cu) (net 1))
 (segment (start 136.398001 83.311999) (end 137.16 82.55) (width 0.25) (layer F.Cu) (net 1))
 (segment (start 127 82.55) (end 128.27 83.82) (width 0.25) (layer F.Cu) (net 1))
 (segment (start 146.558001 83.311999) (end 147.32 82.55) (width 0.25) (layer F.Cu) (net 1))
 (segment (start 146.232999 83.637001) (end 146.558001 83.311999) (width 0.25) (layer F.Cu) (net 1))
 (segment (start 138.247001 83.637001) (end 146.232999 83.637001) (width 0.25) (layer F.Cu) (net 1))
 (segment (start 137.16 82.55) (end 138.247001 83.637001) (width 0.25) (layer F.Cu) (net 1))
 (segment (start 139.46 77.595) (end 139.46 77.47) (width 0.25) (layer F.Cu) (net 1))
 (segment (start 138.36 78.695) (end 139.46 77.595) (width 0.25) (layer F.Cu) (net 1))
 (segment (start 137.16 79.77) (end 138.235 78.695) (width 0.25) (layer F.Cu) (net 1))
 (segment (start 138.235 78.695) (end 138.36 78.695) (width 0.25) (layer F.Cu) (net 1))
 (segment (start 137.16 82.55) (end 137.16 79.77) (width 0.25) (layer F.Cu) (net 1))
 (segment (start 121.158001 88.391999) (end 121.92 87.63) (width 0.25) (layer F.Cu) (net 8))
 (segment (start 120.65 88.9) (end 121.158001 88.391999) (width 0.25) (layer F.Cu) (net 8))
 (segment (start 113.03 88.9) (end 120.65 88.9) (width 0.25) (layer F.Cu) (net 8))
 (segment (start 111.76 87.63) (end 113.03 88.9) (width 0.25) (layer F.Cu) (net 8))
 (segment (start 131.318001 88.391999) (end 132.08 87.63) (width 0.25) (layer F.Cu) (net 8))
 (segment (start 130.81 88.9) (end 131.318001 88.391999) (width 0.25) (layer F.Cu) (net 8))
 (segment (start 123.19 88.9) (end 130.81 88.9) (width 0.25) (layer F.Cu) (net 8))
 (segment (start 121.92 87.63) (end 123.19 88.9) (width 0.25) (layer F.Cu) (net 8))
 (segment (start 141.478001 88.391999) (end 142.24 87.63) (width 0.25) (layer F.Cu) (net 8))
 (segment (start 140.97 88.9) (end 141.478001 88.391999) (width 0.25) (layer F.Cu) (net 8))
 (segment (start 133.35 88.9) (end 140.97 88.9) (width 0.25) (layer F.Cu) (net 8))
 (segment (start 132.08 87.63) (end 133.35 88.9) (width 0.25) (layer F.Cu) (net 8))
 (segment (start 123.36 77.47) (end 124.46 77.47) (width 0.25) (layer F.Cu) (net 8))
 (segment (start 114.730998 77.47) (end 123.36 77.47) (width 0.25) (layer F.Cu) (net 8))
 (segment (start 110.672999 81.527999) (end 114.730998 77.47) (width 0.25) (layer F.Cu) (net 8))
 (segment (start 110.672999 86.542999) (end 110.672999 81.527999) (width 0.25) (layer F.Cu) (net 8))
 (segment (start 111.76 87.63) (end 110.672999 86.542999) (width 0.25) (layer F.Cu) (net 8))
 (segment (start 121.158001 85.851999) (end 121.92 85.09) (width 0.25) (layer F.Cu) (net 9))
 (segment (start 120.65 86.36) (end 121.158001 85.851999) (width 0.25) (layer F.Cu) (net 9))
 (segment (start 113.03 86.36) (end 120.65 86.36) (width 0.25) (layer F.Cu) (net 9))
 (segment (start 111.76 85.09) (end 113.03 86.36) (width 0.25) (layer F.Cu) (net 9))
 (segment (start 131.318001 85.851999) (end 132.08 85.09) (width 0.25) (layer F.Cu) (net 9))
 (segment (start 130.81 86.36) (end 131.318001 85.851999) (width 0.25) (layer F.Cu) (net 9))
 (segment (start 123.19 86.36) (end 130.81 86.36) (width 0.25) (layer F.Cu) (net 9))
 (segment (start 121.92 85.09) (end 123.19 86.36) (width 0.25) (layer F.Cu) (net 9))
 (segment (start 141.478001 85.851999) (end 142.24 85.09) (width 0.25) (layer F.Cu) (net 9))
 (segment (start 140.97 86.36) (end 141.478001 85.851999) (width 0.25) (layer F.Cu) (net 9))
 (segment (start 133.35 86.36) (end 140.97 86.36) (width 0.25) (layer F.Cu) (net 9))
 (segment (start 132.08 85.09) (end 133.35 86.36) (width 0.25) (layer F.Cu) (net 9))
 (segment (start 126.96 77.595) (end 126.96 77.47) (width 0.25) (layer F.Cu) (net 9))
 (segment (start 115.387001 81.462999) (end 123.092001 81.462999) (width 0.25) (layer F.Cu) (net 9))
 (segment (start 123.092001 81.462999) (end 126.96 77.595) (width 0.25) (layer F.Cu) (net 9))
 (segment (start 111.76 85.09) (end 115.387001 81.462999) (width 0.25) (layer F.Cu) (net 9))
 (segment (start 147.365 97.79) (end 153.715 91.44) (width 0.25) (layer F.Cu) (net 18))
 (segment (start 121.92 97.79) (end 147.365 97.79) (width 0.25) (layer F.Cu) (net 18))
 (segment (start 153.715 91.44) (end 154.94 91.44) (width 0.25) (layer F.Cu) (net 18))
 (segment (start 116.84 92.71) (end 121.92 97.79) (width 0.25) (layer F.Cu) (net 18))
 (segment (start 106.805 83.94) (end 106.68 83.94) (width 0.25) (layer B.Cu) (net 19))
 (segment (start 109.042001 86.177001) (end 106.805 83.94) (width 0.25) (layer B.Cu) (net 19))
 (segment (start 112.847001 86.177001) (end 109.042001 86.177001) (width 0.25) (layer B.Cu) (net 19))
 (segment (start 116.84 90.17) (end 112.847001 86.177001) (width 0.25) (layer B.Cu) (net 19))
 (segment (start 106.805 86.44) (end 106.68 86.44) (width 0.25) (layer B.Cu) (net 14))
 (segment (start 105.37999 85.26499) (end 106.555 86.44) (width 0.25) (layer B.Cu) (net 14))
 (segment (start 107.291705 82.76499) (end 106.068295 82.76499) (width 0.25) (layer B.Cu) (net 14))
 (segment (start 105.37999 83.453295) (end 105.37999 85.26499) (width 0.25) (layer B.Cu) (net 14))
 (segment (start 106.068295 82.76499) (end 105.37999 83.453295) (width 0.25) (layer B.Cu) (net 14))
 (segment (start 108.529714 84.002999) (end 107.291705 82.76499) (width 0.25) (layer B.Cu) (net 14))
 (segment (start 112.281761 84.002999) (end 108.529714 84.002999) (width 0.25) (layer B.Cu) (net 14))
 (segment (start 112.847001 85.245763) (end 112.847001 84.568239) (width 0.25) (layer B.Cu) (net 14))
 (segment (start 112.847001 84.568239) (end 112.281761 84.002999) (width 0.25) (layer B.Cu) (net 14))
 (segment (start 116.318239 88.717001) (end 112.847001 85.245763) (width 0.25) (layer B.Cu) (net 14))
 (segment (start 106.555 86.44) (end 106.68 86.44) (width 0.25) (layer B.Cu) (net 14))
 (segment (start 117.290591 88.717001) (end 116.318239 88.717001) (width 0.25) (layer B.Cu) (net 14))
 (segment (start 117.923599 89.350009) (end 117.290591 88.717001) (width 0.25) (layer B.Cu) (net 14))
 (segment (start 119.491248 89.35001) (end 117.923599 89.350009) (width 0.25) (layer B.Cu) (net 14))
 (segment (start 121.398239 91.257001) (end 119.491248 89.35001) (width 0.25) (layer B.Cu) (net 14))
 (segment (start 122.441761 91.257001) (end 121.398239 91.257001) (width 0.25) (layer B.Cu) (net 14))
 (segment (start 123.528762 90.17) (end 122.441761 91.257001) (width 0.25) (layer B.Cu) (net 14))
 (segment (start 127 90.17) (end 123.528762 90.17) (width 0.25) (layer B.Cu) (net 14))
 (segment (start 154.815 88.94) (end 154.94 88.94) (width 0.25) (layer F.Cu) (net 15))
 (segment (start 147.235 96.52) (end 154.815 88.94) (width 0.25) (layer F.Cu) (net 15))
 (segment (start 130.81 96.52) (end 147.235 96.52) (width 0.25) (layer F.Cu) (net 15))
 (segment (start 127 92.71) (end 130.81 96.52) (width 0.25) (layer F.Cu) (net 15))
 (segment (start 151.099999 87.615001) (end 152.275 86.44) (width 0.25) (layer F.Cu) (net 12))
 (segment (start 146.388762 95.25) (end 151.099999 90.538763) (width 0.25) (layer F.Cu) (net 12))
 (segment (start 152.275 86.44) (end 152.4 86.44) (width 0.25) (layer F.Cu) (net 12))
 (segment (start 151.099999 90.538763) (end 151.099999 87.615001) (width 0.25) (layer F.Cu) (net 12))
 (segment (start 139.7 95.25) (end 146.388762 95.25) (width 0.25) (layer F.Cu) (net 12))
 (segment (start 137.16 92.71) (end 139.7 95.25) (width 0.25) (layer F.Cu) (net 12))
 (segment (start 152.275 86.44) (end 154.94 86.44) (width 0.25) (layer F.Cu) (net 12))
 (segment (start 106.805 88.94) (end 106.68 88.94) (width 0.25) (layer B.Cu) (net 13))
 (segment (start 109.22 91.355) (end 106.805 88.94) (width 0.25) (layer B.Cu) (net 13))
 (segment (start 109.22 91.778762) (end 109.22 91.355) (width 0.25) (layer B.Cu) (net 13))
 (segment (start 111.238239 93.797001) (end 109.22 91.778762) (width 0.25) (layer B.Cu) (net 13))
 (segment (start 133.532999 93.797001) (end 111.238239 93.797001) (width 0.25) (layer B.Cu) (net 13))
 (segment (start 137.16 90.17) (end 133.532999 93.797001) (width 0.25) (layer B.Cu) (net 13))
 (segment (start 107.905 91.44) (end 106.68 91.44) (width 0.25) (layer B.Cu) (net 4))
 (segment (start 110.712011 94.247011) (end 107.905 91.44) (width 0.25) (layer B.Cu) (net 4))
 (segment (start 143.242989 94.247011) (end 110.712011 94.247011) (width 0.25) (layer B.Cu) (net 4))
 (segment (start 147.32 90.17) (end 143.242989 94.247011) (width 0.25) (layer B.Cu) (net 4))
 (segment (start 152.275 83.94) (end 152.4 83.94) (width 0.25) (layer F.Cu) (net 5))
 (segment (start 148.407001 87.807999) (end 152.275 83.94) (width 0.25) (layer F.Cu) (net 5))
 (segment (start 148.407001 91.622999) (end 148.407001 87.807999) (width 0.25) (layer F.Cu) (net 5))
 (segment (start 147.32 92.71) (end 148.407001 91.622999) (width 0.25) (layer F.Cu) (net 5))
 (segment (start 152.4 83.94) (end 154.94 83.94) (width 0.25) (layer F.Cu) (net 5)))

